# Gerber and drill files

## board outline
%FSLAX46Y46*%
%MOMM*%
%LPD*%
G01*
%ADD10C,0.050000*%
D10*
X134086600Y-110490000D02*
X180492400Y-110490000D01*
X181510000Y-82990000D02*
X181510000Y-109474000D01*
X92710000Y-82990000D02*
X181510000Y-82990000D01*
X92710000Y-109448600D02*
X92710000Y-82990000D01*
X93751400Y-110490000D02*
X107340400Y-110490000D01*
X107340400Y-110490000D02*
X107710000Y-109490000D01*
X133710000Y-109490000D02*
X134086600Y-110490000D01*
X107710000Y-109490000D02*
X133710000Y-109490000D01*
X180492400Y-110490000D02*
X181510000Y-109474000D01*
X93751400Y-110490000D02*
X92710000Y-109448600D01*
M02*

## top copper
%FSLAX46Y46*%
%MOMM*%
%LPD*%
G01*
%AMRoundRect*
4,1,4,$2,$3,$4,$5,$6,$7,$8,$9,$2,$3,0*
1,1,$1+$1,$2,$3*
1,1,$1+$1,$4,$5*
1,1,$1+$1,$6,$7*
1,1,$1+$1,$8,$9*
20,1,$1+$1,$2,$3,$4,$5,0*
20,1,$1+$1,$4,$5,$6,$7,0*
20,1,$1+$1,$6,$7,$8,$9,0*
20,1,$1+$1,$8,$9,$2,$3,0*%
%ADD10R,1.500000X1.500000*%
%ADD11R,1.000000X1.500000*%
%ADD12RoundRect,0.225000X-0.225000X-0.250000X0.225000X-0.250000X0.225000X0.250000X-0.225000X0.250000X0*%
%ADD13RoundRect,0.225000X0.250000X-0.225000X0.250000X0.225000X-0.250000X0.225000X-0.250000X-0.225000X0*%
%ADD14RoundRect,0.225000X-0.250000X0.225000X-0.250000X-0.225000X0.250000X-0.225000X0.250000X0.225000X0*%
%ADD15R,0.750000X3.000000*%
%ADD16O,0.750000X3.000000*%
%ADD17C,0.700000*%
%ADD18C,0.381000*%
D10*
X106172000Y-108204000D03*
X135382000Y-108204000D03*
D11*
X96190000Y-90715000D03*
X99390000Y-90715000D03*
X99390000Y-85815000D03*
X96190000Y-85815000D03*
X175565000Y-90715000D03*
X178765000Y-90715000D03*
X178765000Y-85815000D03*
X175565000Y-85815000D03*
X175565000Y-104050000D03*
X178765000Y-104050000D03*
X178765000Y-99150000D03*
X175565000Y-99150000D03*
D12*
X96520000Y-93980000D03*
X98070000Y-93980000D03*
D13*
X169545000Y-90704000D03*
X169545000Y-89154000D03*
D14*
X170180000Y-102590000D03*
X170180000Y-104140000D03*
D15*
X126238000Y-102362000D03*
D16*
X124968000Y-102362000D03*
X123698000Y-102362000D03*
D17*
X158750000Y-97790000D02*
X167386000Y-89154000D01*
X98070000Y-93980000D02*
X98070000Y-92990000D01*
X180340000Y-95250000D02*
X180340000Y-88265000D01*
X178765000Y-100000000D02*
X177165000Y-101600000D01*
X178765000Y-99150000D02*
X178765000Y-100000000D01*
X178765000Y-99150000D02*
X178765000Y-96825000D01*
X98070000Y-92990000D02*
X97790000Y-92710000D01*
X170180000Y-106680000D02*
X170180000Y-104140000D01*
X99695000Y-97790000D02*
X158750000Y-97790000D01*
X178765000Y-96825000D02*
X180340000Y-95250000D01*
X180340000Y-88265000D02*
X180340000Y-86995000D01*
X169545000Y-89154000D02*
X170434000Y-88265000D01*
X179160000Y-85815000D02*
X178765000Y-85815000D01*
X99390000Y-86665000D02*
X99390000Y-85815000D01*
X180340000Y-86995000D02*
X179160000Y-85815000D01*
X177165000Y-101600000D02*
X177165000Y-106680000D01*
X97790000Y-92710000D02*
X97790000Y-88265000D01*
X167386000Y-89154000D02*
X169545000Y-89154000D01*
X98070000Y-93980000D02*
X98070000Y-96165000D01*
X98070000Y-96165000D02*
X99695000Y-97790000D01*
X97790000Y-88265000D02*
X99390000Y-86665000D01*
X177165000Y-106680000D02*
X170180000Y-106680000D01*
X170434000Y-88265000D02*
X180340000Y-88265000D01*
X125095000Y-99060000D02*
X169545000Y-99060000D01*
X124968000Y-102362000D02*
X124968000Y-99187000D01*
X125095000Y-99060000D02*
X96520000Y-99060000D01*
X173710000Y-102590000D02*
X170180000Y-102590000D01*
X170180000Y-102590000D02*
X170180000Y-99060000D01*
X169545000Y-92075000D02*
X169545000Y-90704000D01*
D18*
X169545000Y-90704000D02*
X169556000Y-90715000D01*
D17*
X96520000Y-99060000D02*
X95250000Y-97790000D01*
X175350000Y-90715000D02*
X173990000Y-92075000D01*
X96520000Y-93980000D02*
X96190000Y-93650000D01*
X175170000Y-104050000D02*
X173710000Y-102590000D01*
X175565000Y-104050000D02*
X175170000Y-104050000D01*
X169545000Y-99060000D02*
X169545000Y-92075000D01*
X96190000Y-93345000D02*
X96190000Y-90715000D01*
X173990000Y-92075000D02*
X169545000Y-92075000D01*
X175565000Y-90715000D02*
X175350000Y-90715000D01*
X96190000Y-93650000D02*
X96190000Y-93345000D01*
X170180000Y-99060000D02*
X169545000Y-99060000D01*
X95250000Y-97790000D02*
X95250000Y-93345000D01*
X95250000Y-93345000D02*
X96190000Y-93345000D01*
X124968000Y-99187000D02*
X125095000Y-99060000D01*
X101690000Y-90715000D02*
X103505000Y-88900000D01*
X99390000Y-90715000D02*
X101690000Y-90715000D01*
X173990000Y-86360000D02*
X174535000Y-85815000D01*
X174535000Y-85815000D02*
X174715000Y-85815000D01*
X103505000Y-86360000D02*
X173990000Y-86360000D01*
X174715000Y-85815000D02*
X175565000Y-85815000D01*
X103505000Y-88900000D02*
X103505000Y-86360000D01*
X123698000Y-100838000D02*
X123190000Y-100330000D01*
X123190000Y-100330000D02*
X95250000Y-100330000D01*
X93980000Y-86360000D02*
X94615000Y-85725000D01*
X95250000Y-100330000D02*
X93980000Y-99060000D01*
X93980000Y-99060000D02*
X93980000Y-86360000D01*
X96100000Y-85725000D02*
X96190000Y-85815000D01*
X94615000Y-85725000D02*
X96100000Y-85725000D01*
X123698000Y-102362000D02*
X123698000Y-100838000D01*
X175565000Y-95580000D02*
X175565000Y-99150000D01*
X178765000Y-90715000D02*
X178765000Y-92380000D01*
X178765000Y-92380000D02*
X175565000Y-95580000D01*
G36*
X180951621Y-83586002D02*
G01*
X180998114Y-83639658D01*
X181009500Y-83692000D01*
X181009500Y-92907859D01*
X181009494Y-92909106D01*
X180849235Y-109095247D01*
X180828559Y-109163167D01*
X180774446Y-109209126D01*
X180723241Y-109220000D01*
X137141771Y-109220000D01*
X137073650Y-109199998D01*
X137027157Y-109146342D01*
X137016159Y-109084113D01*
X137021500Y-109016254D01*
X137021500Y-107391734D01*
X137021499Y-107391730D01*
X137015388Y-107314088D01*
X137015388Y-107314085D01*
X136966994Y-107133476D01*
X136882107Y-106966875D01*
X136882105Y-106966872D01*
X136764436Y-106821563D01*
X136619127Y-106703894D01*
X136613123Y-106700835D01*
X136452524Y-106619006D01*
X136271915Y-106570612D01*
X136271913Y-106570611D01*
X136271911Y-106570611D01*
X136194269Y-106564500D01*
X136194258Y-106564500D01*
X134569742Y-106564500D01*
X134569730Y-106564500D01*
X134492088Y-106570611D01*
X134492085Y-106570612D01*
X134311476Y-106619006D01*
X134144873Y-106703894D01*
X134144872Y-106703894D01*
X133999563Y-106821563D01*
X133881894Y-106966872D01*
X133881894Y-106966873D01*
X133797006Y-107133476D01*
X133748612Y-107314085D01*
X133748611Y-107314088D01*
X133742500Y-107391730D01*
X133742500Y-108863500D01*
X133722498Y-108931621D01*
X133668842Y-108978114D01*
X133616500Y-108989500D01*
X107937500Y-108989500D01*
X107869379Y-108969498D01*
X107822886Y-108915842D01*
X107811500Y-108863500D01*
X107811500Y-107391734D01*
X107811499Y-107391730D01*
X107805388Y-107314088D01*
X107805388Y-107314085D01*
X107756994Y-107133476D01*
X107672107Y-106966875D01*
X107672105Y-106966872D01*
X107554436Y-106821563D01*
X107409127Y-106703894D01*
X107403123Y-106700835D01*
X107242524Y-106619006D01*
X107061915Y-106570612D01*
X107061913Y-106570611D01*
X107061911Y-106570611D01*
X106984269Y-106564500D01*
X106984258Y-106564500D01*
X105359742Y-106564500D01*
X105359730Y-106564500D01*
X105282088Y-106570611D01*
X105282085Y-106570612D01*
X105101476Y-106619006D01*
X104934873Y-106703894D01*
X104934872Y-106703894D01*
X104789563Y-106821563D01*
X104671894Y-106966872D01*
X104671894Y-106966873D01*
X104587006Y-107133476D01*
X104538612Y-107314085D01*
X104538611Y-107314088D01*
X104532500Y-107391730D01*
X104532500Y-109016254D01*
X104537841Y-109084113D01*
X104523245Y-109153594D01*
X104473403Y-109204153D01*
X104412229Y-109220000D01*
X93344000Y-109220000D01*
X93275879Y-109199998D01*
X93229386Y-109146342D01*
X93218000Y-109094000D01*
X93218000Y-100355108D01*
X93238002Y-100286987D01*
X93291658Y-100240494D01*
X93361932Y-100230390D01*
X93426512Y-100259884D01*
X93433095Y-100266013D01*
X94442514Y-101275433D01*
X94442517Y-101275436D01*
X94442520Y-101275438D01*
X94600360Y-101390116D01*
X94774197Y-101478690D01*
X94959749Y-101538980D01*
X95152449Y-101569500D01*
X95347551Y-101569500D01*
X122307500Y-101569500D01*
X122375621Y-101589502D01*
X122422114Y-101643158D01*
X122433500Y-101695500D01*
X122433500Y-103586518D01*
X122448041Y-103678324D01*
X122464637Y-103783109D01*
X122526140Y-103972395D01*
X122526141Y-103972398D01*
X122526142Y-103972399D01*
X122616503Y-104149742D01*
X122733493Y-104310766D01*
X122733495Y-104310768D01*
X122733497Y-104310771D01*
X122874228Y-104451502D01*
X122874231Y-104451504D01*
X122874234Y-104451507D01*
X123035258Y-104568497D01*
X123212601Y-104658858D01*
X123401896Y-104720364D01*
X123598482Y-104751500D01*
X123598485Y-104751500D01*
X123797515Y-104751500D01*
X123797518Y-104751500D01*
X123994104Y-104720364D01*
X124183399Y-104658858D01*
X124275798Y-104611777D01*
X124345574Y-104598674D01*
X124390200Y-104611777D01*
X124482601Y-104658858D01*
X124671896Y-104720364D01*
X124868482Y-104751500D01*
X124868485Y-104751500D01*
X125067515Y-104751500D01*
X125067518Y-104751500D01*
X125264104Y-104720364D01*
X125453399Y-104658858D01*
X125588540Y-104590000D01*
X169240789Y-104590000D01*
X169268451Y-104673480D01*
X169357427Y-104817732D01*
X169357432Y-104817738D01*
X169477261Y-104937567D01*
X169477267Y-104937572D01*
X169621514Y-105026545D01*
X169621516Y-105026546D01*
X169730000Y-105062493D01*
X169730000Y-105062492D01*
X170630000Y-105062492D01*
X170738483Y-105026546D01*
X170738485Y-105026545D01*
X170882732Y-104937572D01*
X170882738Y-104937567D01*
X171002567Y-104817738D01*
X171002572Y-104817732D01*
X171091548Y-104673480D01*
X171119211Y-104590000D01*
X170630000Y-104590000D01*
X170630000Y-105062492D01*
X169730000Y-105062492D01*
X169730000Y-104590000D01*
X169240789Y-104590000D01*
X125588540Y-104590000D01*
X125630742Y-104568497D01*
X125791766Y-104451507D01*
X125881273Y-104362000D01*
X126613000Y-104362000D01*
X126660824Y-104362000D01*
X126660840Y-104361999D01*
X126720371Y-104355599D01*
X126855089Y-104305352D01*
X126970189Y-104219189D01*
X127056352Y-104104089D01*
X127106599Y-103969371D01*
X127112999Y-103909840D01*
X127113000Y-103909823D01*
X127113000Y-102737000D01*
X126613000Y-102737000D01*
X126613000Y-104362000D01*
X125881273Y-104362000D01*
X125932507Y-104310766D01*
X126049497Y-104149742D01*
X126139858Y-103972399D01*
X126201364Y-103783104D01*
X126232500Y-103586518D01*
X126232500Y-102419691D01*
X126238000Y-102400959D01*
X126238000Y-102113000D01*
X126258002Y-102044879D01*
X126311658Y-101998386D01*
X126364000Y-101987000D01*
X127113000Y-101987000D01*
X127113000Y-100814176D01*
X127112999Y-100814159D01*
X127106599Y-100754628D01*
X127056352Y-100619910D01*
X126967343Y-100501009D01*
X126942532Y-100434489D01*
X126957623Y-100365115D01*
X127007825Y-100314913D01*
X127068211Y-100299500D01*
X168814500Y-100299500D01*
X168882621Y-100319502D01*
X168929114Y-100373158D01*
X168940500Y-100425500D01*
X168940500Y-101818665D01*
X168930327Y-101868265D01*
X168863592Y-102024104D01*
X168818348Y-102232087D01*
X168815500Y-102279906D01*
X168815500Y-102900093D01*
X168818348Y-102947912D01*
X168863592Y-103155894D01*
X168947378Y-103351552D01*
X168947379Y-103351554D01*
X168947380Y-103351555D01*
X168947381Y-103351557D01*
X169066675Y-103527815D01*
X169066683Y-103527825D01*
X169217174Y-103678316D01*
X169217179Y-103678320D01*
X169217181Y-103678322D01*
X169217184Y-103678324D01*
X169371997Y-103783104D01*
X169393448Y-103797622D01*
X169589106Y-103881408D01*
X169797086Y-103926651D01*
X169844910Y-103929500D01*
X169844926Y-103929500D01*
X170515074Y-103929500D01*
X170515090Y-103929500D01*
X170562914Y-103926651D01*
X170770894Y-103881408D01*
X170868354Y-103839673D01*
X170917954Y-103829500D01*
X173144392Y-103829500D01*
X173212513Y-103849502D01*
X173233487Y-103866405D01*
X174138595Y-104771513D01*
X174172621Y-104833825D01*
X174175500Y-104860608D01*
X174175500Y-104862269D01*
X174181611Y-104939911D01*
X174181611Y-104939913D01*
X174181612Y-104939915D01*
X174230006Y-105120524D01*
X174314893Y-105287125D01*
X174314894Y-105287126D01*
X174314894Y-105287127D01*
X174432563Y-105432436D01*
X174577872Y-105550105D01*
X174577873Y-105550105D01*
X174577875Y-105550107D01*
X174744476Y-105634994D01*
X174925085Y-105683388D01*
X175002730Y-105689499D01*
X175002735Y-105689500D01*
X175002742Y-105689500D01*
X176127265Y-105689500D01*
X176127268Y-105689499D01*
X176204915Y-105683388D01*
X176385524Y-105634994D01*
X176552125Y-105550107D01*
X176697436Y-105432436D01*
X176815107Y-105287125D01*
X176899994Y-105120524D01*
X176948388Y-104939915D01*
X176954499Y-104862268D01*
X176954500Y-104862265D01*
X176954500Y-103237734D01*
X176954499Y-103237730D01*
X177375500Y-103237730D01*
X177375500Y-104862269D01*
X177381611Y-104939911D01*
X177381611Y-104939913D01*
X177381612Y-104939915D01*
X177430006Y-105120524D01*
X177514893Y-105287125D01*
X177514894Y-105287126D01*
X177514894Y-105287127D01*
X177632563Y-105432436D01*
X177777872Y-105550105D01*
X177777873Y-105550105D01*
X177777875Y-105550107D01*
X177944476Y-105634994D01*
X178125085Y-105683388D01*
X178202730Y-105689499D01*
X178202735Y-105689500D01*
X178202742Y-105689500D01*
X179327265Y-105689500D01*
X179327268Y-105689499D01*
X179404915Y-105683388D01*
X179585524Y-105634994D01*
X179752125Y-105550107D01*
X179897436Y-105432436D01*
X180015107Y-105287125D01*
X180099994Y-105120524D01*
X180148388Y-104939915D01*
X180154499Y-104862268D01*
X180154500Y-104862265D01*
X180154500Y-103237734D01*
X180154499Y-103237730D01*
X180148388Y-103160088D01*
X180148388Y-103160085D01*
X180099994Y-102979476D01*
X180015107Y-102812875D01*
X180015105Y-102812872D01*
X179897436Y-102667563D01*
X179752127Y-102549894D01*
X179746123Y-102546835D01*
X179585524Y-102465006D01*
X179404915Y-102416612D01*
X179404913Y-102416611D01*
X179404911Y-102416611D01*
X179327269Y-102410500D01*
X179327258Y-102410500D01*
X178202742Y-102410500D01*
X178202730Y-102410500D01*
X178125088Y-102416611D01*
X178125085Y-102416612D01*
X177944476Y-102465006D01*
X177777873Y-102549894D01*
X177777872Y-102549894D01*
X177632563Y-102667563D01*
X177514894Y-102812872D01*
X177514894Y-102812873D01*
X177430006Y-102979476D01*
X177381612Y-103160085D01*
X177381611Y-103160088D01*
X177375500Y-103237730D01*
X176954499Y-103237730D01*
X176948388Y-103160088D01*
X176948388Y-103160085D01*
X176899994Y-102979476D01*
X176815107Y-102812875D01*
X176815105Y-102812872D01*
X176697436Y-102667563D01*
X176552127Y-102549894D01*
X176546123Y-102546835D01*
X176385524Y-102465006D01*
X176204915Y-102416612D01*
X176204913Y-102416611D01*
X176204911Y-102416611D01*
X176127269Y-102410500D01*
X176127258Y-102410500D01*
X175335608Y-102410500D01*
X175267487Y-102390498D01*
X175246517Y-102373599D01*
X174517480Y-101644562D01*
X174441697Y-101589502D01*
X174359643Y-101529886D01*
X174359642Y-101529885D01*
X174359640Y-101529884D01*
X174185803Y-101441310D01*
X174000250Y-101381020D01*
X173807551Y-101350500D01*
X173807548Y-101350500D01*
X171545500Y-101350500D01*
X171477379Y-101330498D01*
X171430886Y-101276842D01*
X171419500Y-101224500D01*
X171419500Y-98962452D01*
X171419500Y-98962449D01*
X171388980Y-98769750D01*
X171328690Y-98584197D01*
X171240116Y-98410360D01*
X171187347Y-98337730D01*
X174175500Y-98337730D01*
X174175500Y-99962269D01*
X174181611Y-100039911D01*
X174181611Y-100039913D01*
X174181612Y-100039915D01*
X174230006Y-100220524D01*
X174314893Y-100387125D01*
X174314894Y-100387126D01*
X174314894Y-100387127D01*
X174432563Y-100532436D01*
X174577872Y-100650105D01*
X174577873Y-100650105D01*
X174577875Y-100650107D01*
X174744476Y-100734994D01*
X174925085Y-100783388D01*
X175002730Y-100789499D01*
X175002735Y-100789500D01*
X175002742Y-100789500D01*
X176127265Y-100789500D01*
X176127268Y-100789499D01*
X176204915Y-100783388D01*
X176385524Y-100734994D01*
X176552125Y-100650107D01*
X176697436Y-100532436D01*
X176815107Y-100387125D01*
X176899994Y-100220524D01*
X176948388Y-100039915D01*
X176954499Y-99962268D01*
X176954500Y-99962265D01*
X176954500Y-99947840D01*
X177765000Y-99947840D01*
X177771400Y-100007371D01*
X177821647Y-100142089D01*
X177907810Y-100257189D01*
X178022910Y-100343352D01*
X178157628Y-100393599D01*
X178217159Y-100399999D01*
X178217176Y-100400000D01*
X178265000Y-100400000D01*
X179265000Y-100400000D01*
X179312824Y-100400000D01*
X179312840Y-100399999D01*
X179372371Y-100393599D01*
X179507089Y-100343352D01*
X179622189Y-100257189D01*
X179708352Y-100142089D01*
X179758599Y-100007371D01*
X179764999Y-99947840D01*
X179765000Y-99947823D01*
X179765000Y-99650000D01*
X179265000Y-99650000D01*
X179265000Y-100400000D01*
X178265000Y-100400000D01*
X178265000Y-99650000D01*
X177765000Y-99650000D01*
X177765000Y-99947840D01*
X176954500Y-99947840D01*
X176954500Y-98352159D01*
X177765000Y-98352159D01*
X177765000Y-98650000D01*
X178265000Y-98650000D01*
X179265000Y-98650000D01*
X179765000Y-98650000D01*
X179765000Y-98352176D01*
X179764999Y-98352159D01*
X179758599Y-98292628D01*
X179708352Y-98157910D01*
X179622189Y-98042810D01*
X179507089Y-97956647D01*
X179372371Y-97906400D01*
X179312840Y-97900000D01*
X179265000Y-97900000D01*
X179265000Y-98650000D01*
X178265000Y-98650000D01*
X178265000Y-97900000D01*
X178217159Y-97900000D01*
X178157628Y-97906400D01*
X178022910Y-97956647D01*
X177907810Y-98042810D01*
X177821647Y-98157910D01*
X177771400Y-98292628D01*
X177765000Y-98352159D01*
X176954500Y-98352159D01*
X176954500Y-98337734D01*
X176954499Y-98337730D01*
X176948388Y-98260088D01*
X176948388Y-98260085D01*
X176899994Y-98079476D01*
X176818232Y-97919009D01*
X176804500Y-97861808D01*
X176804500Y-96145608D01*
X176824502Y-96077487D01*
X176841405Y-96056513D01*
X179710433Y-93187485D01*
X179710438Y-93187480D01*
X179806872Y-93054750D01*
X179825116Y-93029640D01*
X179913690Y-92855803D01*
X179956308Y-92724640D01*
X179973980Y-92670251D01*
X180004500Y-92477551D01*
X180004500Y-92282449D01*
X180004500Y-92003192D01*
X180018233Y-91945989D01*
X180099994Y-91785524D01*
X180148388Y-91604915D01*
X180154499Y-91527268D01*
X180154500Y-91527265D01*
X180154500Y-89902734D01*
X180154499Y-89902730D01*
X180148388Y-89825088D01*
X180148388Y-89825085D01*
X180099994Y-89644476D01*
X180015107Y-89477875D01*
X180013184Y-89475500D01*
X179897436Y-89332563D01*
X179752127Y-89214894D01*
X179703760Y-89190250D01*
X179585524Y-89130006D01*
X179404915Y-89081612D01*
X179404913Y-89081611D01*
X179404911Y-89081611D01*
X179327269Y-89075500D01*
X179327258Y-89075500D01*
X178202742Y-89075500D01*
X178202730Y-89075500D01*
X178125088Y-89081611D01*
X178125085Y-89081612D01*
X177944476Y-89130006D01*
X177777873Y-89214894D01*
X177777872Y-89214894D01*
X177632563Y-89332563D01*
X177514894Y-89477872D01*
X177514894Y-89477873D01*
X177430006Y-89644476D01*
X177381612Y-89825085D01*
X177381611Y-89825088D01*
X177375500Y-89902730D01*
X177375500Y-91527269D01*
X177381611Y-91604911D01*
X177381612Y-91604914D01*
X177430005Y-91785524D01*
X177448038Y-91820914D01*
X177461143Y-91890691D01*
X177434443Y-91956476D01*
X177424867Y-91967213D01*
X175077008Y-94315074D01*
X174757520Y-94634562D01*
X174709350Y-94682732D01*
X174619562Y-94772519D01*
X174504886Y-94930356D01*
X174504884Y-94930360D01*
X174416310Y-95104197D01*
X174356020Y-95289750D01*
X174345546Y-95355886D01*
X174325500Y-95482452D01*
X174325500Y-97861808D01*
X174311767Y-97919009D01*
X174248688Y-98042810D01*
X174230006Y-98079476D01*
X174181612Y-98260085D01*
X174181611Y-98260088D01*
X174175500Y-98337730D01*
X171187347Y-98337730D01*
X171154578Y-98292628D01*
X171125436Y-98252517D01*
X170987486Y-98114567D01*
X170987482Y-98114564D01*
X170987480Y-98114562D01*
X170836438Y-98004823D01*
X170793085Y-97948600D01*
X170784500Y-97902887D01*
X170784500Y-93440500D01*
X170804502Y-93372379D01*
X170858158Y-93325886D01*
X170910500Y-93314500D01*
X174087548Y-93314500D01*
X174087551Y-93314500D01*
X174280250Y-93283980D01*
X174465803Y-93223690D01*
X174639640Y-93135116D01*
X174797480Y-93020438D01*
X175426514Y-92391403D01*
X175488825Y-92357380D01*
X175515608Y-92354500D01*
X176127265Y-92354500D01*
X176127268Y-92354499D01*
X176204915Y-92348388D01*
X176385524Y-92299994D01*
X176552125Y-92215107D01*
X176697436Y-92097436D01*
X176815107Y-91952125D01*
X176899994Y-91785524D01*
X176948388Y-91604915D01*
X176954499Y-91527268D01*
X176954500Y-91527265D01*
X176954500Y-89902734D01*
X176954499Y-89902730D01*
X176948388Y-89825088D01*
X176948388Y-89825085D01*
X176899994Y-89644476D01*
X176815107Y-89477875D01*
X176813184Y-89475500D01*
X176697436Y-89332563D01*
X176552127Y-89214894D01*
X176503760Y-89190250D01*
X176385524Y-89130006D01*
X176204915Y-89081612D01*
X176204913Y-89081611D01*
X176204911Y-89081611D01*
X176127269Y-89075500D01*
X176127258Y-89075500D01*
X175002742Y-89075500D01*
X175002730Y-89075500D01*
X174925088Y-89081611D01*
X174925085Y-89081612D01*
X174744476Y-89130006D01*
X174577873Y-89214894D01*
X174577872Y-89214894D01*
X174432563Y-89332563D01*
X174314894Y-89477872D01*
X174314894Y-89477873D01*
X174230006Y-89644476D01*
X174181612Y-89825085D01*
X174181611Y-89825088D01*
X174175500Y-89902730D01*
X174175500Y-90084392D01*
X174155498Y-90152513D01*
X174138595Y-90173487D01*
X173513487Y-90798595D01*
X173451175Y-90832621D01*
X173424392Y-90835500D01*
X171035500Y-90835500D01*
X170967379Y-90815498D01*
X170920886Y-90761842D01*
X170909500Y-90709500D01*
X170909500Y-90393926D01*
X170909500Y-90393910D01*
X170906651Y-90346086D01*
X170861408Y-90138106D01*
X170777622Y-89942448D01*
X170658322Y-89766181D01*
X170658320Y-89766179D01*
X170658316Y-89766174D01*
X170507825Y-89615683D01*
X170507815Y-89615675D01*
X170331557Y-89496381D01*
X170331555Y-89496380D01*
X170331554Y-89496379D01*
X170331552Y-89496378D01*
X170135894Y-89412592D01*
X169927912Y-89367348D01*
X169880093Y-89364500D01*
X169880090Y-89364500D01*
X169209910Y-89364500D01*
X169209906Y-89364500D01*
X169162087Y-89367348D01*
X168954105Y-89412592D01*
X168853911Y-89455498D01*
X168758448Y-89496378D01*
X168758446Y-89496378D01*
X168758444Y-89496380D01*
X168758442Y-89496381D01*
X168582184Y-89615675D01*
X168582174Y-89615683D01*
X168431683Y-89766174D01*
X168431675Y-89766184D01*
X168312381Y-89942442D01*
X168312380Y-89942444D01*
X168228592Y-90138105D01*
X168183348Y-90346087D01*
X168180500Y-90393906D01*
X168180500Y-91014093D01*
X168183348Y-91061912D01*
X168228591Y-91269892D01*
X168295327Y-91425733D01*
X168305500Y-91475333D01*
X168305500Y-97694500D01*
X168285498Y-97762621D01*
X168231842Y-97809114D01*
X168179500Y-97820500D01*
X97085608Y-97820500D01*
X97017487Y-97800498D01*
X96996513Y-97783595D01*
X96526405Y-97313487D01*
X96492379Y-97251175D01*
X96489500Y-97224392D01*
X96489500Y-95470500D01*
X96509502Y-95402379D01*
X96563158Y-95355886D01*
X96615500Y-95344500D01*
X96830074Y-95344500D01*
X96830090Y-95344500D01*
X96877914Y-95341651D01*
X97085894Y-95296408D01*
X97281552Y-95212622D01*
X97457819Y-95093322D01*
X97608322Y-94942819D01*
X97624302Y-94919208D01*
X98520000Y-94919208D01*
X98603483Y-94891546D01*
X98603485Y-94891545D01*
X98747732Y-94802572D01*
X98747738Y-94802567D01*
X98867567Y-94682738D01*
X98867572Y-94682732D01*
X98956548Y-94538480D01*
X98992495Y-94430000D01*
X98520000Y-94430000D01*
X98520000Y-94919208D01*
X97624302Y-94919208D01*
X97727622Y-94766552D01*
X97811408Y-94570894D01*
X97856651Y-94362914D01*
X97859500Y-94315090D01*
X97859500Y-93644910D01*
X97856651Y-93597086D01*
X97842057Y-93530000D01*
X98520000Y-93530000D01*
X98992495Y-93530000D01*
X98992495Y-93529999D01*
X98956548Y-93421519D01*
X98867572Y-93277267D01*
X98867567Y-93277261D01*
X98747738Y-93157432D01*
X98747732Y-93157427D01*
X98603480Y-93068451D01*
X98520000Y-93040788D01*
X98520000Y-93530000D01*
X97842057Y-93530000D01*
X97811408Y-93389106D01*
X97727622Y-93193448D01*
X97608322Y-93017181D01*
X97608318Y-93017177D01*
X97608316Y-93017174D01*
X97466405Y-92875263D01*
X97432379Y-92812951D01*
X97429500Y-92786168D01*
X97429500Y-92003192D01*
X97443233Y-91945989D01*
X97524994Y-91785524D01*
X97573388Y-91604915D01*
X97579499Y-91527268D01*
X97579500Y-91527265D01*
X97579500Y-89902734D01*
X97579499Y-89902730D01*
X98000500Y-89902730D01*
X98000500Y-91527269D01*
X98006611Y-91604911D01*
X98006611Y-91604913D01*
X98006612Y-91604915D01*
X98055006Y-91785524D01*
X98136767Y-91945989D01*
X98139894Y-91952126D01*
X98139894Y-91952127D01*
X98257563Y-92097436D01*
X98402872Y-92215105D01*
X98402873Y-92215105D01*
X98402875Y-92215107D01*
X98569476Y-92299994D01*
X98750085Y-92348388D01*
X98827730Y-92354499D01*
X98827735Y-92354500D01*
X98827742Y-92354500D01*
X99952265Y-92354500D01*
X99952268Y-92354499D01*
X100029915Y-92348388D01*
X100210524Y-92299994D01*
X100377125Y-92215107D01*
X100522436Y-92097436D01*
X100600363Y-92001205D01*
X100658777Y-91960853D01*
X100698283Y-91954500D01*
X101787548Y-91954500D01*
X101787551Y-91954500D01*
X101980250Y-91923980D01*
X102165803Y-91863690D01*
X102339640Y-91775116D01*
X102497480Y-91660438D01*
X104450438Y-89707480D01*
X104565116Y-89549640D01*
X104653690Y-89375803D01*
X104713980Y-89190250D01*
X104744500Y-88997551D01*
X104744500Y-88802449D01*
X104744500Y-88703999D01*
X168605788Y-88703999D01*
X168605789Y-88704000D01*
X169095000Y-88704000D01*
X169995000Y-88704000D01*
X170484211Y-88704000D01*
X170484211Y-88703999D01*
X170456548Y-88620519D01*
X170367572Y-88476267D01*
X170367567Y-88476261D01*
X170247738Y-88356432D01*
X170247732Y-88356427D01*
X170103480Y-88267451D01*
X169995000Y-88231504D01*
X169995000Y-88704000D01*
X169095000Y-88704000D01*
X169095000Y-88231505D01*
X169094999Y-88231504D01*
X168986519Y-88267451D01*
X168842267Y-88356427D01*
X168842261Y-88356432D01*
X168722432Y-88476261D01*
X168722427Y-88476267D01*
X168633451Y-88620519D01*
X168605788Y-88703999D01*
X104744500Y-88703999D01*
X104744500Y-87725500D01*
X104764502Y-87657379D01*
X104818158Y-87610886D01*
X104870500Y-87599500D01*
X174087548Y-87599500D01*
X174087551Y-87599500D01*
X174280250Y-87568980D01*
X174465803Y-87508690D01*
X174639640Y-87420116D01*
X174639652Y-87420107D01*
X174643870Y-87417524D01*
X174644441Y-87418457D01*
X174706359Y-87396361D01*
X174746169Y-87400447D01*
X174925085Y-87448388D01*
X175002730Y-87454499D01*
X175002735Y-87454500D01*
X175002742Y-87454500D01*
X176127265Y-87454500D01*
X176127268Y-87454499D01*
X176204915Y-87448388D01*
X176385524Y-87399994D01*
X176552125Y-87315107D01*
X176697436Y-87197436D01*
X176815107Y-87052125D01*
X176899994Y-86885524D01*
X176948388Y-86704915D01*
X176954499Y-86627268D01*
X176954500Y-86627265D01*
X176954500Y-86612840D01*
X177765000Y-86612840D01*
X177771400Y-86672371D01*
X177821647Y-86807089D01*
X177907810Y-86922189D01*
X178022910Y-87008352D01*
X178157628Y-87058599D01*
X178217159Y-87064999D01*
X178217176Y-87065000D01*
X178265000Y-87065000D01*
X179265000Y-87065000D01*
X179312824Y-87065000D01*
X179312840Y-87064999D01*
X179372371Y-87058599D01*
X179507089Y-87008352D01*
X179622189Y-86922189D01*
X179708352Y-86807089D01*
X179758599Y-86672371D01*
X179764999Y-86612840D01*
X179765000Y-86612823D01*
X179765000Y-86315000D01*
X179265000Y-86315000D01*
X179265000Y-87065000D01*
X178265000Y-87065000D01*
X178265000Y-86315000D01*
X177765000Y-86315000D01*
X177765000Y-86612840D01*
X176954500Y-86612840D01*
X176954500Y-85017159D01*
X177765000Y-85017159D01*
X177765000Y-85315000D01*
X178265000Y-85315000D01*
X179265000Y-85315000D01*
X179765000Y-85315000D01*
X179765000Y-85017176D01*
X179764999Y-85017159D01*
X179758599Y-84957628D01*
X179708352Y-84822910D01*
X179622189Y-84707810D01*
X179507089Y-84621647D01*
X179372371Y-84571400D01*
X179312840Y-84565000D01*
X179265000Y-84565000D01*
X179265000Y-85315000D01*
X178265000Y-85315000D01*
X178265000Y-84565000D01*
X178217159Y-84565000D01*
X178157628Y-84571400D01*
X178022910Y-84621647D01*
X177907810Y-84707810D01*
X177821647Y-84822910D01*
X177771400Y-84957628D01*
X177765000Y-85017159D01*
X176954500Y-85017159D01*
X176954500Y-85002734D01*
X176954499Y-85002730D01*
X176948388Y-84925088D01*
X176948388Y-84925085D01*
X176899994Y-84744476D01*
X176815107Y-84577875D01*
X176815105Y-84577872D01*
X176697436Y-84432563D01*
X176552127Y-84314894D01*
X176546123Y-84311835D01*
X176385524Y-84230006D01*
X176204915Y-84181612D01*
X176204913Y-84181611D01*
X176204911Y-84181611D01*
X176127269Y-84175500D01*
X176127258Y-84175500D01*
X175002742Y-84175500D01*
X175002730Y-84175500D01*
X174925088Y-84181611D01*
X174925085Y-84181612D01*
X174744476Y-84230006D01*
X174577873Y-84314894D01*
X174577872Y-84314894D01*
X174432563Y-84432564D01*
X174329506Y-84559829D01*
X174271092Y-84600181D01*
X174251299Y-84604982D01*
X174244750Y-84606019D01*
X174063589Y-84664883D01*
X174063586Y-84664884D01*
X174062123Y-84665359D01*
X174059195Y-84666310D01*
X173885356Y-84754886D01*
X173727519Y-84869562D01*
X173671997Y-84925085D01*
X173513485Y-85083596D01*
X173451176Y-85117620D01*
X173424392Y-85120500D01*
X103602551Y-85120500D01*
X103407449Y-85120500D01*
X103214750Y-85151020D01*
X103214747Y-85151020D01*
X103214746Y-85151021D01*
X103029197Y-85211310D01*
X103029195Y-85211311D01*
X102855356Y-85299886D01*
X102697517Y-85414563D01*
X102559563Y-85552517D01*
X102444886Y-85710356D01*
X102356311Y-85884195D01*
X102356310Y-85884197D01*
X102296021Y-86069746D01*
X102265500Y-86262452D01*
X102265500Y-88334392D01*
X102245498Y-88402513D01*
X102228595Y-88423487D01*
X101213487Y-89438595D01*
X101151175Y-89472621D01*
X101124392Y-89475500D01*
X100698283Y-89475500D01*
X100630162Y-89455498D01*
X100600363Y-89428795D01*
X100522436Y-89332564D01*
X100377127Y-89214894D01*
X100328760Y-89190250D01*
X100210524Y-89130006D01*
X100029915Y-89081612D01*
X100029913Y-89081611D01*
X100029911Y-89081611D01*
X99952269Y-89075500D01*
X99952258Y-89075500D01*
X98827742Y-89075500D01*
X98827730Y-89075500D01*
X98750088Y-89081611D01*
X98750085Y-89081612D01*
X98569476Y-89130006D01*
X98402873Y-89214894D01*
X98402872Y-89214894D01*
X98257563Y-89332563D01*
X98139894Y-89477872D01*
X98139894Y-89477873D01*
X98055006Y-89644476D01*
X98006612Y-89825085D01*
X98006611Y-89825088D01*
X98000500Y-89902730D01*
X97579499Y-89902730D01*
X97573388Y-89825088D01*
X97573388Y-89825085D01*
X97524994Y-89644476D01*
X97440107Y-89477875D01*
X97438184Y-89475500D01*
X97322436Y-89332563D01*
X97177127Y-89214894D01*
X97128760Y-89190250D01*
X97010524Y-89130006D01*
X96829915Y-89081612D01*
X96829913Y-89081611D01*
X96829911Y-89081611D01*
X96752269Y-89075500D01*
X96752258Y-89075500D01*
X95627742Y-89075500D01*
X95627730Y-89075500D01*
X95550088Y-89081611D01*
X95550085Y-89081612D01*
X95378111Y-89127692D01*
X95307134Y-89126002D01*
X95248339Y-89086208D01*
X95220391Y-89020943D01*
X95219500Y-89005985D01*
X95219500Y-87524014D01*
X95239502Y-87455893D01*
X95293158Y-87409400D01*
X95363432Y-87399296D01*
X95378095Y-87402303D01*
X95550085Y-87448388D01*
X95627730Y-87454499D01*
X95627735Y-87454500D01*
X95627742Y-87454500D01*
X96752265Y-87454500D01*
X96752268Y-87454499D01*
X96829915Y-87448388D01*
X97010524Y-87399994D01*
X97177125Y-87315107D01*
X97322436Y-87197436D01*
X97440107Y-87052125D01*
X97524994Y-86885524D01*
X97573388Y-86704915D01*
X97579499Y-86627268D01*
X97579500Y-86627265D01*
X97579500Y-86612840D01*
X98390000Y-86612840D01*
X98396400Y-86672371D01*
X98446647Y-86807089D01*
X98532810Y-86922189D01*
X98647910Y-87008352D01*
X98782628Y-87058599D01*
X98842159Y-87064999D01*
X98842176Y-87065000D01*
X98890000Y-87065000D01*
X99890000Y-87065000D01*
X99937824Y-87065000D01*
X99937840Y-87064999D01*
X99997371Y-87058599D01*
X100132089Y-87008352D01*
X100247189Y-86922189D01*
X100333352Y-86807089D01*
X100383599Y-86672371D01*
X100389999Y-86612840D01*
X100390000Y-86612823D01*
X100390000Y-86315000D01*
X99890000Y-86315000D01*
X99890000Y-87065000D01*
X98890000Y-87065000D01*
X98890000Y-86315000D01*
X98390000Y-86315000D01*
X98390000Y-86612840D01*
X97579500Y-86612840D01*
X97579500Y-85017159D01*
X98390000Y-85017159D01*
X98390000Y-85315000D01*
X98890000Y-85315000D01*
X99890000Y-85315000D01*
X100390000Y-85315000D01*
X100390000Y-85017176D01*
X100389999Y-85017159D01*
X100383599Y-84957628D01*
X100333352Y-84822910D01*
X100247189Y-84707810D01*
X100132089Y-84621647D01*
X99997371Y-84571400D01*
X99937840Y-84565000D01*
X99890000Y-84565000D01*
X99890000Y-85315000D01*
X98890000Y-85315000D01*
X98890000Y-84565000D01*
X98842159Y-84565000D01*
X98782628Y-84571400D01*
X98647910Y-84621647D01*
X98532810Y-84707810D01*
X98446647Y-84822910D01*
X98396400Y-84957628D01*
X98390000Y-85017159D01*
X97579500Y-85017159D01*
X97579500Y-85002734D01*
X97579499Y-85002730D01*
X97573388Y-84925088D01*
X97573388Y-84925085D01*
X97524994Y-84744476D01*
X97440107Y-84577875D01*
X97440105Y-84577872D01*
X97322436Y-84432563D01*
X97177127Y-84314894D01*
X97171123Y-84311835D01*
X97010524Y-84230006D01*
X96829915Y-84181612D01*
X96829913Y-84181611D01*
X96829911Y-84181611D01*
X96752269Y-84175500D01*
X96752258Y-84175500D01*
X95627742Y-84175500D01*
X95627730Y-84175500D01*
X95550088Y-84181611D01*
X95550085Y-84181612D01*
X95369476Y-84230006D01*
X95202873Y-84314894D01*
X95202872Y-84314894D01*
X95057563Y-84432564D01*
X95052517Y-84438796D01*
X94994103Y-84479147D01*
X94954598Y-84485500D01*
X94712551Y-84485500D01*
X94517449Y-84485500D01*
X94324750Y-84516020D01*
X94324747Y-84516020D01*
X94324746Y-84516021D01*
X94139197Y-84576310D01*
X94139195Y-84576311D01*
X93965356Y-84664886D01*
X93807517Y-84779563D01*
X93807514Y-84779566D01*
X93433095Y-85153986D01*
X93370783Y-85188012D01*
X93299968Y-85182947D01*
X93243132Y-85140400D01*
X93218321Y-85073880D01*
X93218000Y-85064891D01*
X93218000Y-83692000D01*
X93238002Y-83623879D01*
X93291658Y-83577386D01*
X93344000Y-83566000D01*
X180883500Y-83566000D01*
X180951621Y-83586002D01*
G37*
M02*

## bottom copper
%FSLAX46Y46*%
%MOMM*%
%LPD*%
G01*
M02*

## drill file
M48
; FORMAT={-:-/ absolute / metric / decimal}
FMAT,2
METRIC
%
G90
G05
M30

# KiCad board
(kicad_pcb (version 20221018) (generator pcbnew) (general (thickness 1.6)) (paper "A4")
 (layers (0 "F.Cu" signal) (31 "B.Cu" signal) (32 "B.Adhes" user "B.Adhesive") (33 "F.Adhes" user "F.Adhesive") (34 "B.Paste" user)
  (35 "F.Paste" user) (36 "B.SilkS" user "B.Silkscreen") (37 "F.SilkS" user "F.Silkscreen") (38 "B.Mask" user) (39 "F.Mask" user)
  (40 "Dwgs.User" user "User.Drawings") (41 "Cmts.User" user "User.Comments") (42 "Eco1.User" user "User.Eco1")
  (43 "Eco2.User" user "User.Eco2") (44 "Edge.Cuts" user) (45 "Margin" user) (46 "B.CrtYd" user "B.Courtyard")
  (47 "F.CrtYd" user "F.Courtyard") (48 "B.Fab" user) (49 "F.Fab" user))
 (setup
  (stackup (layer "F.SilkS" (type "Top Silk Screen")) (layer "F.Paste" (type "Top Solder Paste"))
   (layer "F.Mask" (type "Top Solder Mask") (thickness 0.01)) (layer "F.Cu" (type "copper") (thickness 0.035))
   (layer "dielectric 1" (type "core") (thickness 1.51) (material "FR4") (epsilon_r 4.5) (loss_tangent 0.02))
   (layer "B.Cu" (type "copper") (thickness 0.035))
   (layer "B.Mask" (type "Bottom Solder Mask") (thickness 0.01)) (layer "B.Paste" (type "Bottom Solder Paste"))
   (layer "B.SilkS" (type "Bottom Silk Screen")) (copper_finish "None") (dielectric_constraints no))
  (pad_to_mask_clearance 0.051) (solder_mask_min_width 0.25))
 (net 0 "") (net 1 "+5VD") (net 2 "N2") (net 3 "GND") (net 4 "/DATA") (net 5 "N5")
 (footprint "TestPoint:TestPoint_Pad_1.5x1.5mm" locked (layer "F.Cu") (at 106.172 108.204)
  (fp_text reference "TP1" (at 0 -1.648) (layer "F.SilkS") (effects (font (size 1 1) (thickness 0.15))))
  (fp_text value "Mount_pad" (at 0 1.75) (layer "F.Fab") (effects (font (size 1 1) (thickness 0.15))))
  (pad "1" smd rect locked (at 0 0) (size 1.5 1.5) (layers "F.Cu" "F.Mask")))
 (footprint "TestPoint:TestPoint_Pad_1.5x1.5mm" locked (layer "F.Cu") (at 135.382 108.204)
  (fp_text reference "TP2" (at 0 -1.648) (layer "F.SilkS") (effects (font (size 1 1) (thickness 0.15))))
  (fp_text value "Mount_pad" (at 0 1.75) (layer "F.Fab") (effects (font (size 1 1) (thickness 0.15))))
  (pad "1" smd rect locked (at 0 0) (size 1.5 1.5) (layers "F.Cu" "F.Mask")))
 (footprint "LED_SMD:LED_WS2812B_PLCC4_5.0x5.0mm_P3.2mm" (layer "F.Cu") (at 97.79 88.265 90)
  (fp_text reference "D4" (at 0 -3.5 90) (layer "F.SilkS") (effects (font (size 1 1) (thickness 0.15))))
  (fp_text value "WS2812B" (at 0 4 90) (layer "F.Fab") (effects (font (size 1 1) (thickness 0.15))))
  (pad "1" smd rect (at -2.45 -1.6 90) (size 1.5 1) (layers "F.Cu" "F.Paste" "F.Mask") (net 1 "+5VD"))
  (pad "2" smd rect (at -2.45 1.6 90) (size 1.5 1) (layers "F.Cu" "F.Paste" "F.Mask") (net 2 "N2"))
  (pad "3" smd rect (at 2.45 1.6 90) (size 1.5 1) (layers "F.Cu" "F.Paste" "F.Mask") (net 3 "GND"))
  (pad "4" smd rect (at 2.45 -1.6 90) (size 1.5 1) (layers "F.Cu" "F.Paste" "F.Mask") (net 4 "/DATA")))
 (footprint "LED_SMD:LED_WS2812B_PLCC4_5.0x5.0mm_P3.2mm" (layer "F.Cu") (at 177.165 88.265 90)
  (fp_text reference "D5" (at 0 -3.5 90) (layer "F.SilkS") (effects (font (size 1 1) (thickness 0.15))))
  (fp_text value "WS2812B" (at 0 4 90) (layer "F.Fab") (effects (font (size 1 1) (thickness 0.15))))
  (pad "1" smd rect (at -2.45 -1.6 90) (size 1.5 1) (layers "F.Cu" "F.Paste" "F.Mask") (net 1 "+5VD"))
  (pad "2" smd rect (at -2.45 1.6 90) (size 1.5 1) (layers "F.Cu" "F.Paste" "F.Mask") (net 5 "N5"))
  (pad "3" smd rect (at 2.45 1.6 90) (size 1.5 1) (layers "F.Cu" "F.Paste" "F.Mask") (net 3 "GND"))
  (pad "4" smd rect (at 2.45 -1.6 90) (size 1.5 1) (layers "F.Cu" "F.Paste" "F.Mask") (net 2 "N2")))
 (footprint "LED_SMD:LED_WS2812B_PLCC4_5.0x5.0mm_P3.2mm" (layer "F.Cu") (at 177.165 101.6 90)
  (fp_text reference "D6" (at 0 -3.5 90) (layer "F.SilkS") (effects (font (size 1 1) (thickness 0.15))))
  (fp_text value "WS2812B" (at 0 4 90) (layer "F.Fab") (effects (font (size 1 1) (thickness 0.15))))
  (pad "1" smd rect (at -2.45 -1.6 90) (size 1.5 1) (layers "F.Cu" "F.Paste" "F.Mask") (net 1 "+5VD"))
  (pad "2" smd rect (at -2.45 1.6 90) (size 1.5 1) (layers "F.Cu" "F.Paste" "F.Mask"))
  (pad "3" smd rect (at 2.45 1.6 90) (size 1.5 1) (layers "F.Cu" "F.Paste" "F.Mask") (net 3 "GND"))
  (pad "4" smd rect (at 2.45 -1.6 90) (size 1.5 1) (layers "F.Cu" "F.Paste" "F.Mask") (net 5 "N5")))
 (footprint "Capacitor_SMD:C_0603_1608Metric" (layer "F.Cu") (at 97.295 93.98)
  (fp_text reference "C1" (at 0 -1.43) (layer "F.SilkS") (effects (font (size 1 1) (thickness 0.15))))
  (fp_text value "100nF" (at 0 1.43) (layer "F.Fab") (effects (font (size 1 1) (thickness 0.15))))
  (pad "1" smd roundrect (at -0.775 0) (size 0.9 0.95) (layers "F.Cu" "F.Paste" "F.Mask") (roundrect_rratio 0.25) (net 1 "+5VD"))
  (pad "2" smd roundrect (at 0.775 0) (size 0.9 0.95) (layers "F.Cu" "F.Paste" "F.Mask") (roundrect_rratio 0.25) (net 3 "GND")))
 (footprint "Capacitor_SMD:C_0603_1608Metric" (layer "F.Cu") (at 169.545 89.929 90)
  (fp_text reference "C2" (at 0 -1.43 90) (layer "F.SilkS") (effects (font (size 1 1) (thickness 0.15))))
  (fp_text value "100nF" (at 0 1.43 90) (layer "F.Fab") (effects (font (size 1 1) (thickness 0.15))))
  (pad "1" smd roundrect (at -0.775 0 90) (size 0.9 0.95) (layers "F.Cu" "F.Paste" "F.Mask") (roundrect_rratio 0.25) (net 1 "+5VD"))
  (pad "2" smd roundrect (at 0.775 0 90) (size 0.9 0.95) (layers "F.Cu" "F.Paste" "F.Mask") (roundrect_rratio 0.25) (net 3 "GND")))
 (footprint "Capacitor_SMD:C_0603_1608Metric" (layer "F.Cu") (at 170.18 103.365 -90)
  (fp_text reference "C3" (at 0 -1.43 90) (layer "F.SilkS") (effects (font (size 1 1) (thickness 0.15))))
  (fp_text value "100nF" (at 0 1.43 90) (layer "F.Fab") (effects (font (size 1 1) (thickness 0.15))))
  (pad "1" smd roundrect (at -0.775 0 270) (size 0.9 0.95) (layers "F.Cu" "F.Paste" "F.Mask") (roundrect_rratio 0.25) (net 1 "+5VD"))
  (pad "2" smd roundrect (at 0.775 0 270) (size 0.9 0.95) (layers "F.Cu" "F.Paste" "F.Mask") (roundrect_rratio 0.25) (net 3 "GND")))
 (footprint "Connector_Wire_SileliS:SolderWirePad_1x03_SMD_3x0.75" (layer "F.Cu") (at 124.9553 105.3493 180)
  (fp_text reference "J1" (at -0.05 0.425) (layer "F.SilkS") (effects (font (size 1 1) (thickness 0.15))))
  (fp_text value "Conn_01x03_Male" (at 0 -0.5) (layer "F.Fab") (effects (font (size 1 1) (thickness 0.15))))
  (pad "1" smd rect (at -1.2827 2.9873 180) (size 0.75 3) (layers "F.Cu" "F.Mask") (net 3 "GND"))
  (pad "2" smd oval (at -0.0127 2.9873 180) (size 0.75 3) (layers "F.Cu" "F.Mask") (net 1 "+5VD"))
  (pad "3" smd oval (at 1.2573 2.9873 180) (size 0.75 3) (layers "F.Cu" "F.Mask") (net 4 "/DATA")))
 (gr_line (start 134.0866 110.49) (end 180.4924 110.49) (stroke (width 0.05) (type solid)) (layer "Edge.Cuts"))
 (gr_line (start 181.51 82.99) (end 181.51 109.474) (stroke (width 0.05) (type solid)) (layer "Edge.Cuts"))
 (gr_line (start 92.71 82.99) (end 181.51 82.99) (stroke (width 0.05) (type solid)) (layer "Edge.Cuts"))
 (gr_line (start 92.71 109.4486) (end 92.71 82.99) (stroke (width 0.05) (type solid)) (layer "Edge.Cuts"))
 (gr_line (start 93.7514 110.49) (end 107.3404 110.49) (stroke (width 0.05) (type solid)) (layer "Edge.Cuts"))
 (gr_line (start 107.3404 110.49) (end 107.71 109.49) (stroke (width 0.05) (type solid)) (layer "Edge.Cuts"))
 (gr_line (start 133.71 109.49) (end 134.0866 110.49) (stroke (width 0.05) (type solid)) (layer "Edge.Cuts"))
 (gr_line (start 107.71 109.49) (end 133.71 109.49) (stroke (width 0.05) (type solid)) (layer "Edge.Cuts"))
 (gr_line (start 180.4924 110.49) (end 181.51 109.474) (stroke (width 0.05) (type solid)) (layer "Edge.Cuts"))
 (gr_line (start 93.7514 110.49) (end 92.71 109.4486) (stroke (width 0.05) (type solid)) (layer "Edge.Cuts"))
 (segment (start 158.75 97.79) (end 167.386 89.154) (width 0.7) (layer "F.Cu") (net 3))
 (segment (start 98.07 93.98) (end 98.07 92.99) (width 0.7) (layer "F.Cu") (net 3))
 (segment (start 180.34 95.25) (end 180.34 88.265) (width 0.7) (layer "F.Cu") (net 3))
 (segment (start 178.765 100) (end 177.165 101.6) (width 0.7) (layer "F.Cu") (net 3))
 (segment (start 178.765 99.15) (end 178.765 100) (width 0.7) (layer "F.Cu") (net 3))
 (segment (start 178.765 99.15) (end 178.765 96.825) (width 0.7) (layer "F.Cu") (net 3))
 (segment (start 98.07 92.99) (end 97.79 92.71) (width 0.7) (layer "F.Cu") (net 3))
 (segment (start 170.18 106.68) (end 170.18 104.14) (width 0.7) (layer "F.Cu") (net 3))
 (segment (start 99.695 97.79) (end 158.75 97.79) (width 0.7) (layer "F.Cu") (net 3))
 (segment (start 178.765 96.825) (end 180.34 95.25) (width 0.7) (layer "F.Cu") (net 3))
 (segment (start 180.34 88.265) (end 180.34 86.995) (width 0.7) (layer "F.Cu") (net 3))
 (segment (start 169.545 89.154) (end 170.434 88.265) (width 0.7) (layer "F.Cu") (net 3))
 (segment (start 179.16 85.815) (end 178.765 85.815) (width 0.7) (layer "F.Cu") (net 3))
 (segment (start 99.39 86.665) (end 99.39 85.815) (width 0.7) (layer "F.Cu") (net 3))
 (segment (start 180.34 86.995) (end 179.16 85.815) (width 0.7) (layer "F.Cu") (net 3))
 (segment (start 177.165 101.6) (end 177.165 106.68) (width 0.7) (layer "F.Cu") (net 3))
 (segment (start 97.79 92.71) (end 97.79 88.265) (width 0.7) (layer "F.Cu") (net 3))
 (segment (start 167.386 89.154) (end 169.545 89.154) (width 0.7) (layer "F.Cu") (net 3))
 (segment (start 98.07 93.98) (end 98.07 96.165) (width 0.7) (layer "F.Cu") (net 3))
 (segment (start 98.07 96.165) (end 99.695 97.79) (width 0.7) (layer "F.Cu") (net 3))
 (segment (start 97.79 88.265) (end 99.39 86.665) (width 0.7) (layer "F.Cu") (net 3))
 (segment (start 177.165 106.68) (end 170.18 106.68) (width 0.7) (layer "F.Cu") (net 3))
 (segment (start 170.434 88.265) (end 180.34 88.265) (width 0.7) (layer "F.Cu") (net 3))
 (segment (start 125.095 99.06) (end 169.545 99.06) (width 0.7) (layer "F.Cu") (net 1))
 (segment (start 124.968 102.362) (end 124.968 99.187) (width 0.7) (layer "F.Cu") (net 1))
 (segment (start 125.095 99.06) (end 96.52 99.06) (width 0.7) (layer "F.Cu") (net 1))
 (segment (start 173.71 102.59) (end 170.18 102.59) (width 0.7) (layer "F.Cu") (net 1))
 (segment (start 170.18 102.59) (end 170.18 99.06) (width 0.7) (layer "F.Cu") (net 1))
 (segment (start 169.545 92.075) (end 169.545 90.704) (width 0.7) (layer "F.Cu") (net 1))
 (segment (start 169.545 90.704) (end 169.556 90.715) (width 0.381) (layer "F.Cu") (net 1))
 (segment (start 96.52 99.06) (end 95.25 97.79) (width 0.7) (layer "F.Cu") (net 1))
 (segment (start 175.35 90.715) (end 173.99 92.075) (width 0.7) (layer "F.Cu") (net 1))
 (segment (start 96.52 93.98) (end 96.19 93.65) (width 0.7) (layer "F.Cu") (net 1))
 (segment (start 175.17 104.05) (end 173.71 102.59) (width 0.7) (layer "F.Cu") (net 1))
 (segment (start 175.565 104.05) (end 175.17 104.05) (width 0.7) (layer "F.Cu") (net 1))
 (segment (start 169.545 99.06) (end 169.545 92.075) (width 0.7) (layer "F.Cu") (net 1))
 (segment (start 96.19 93.345) (end 96.19 90.715) (width 0.7) (layer "F.Cu") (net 1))
 (segment (start 173.99 92.075) (end 169.545 92.075) (width 0.7) (layer "F.Cu") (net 1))
 (segment (start 175.565 90.715) (end 175.35 90.715) (width 0.7) (layer "F.Cu") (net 1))
 (segment (start 96.19 93.65) (end 96.19 93.345) (width 0.7) (layer "F.Cu") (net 1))
 (segment (start 170.18 99.06) (end 169.545 99.06) (width 0.7) (layer "F.Cu") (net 1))
 (segment (start 95.25 97.79) (end 95.25 93.345) (width 0.7) (layer "F.Cu") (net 1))
 (segment (start 95.25 93.345) (end 96.19 93.345) (width 0.7) (layer "F.Cu") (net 1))
 (segment (start 124.968 99.187) (end 125.095 99.06) (width 0.7) (layer "F.Cu") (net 1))
 (segment (start 101.69 90.715) (end 103.505 88.9) (width 0.7) (layer "F.Cu") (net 2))
 (segment (start 99.39 90.715) (end 101.69 90.715) (width 0.7) (layer "F.Cu") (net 2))
 (segment (start 173.99 86.36) (end 174.535 85.815) (width 0.7) (layer "F.Cu") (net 2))
 (segment (start 174.535 85.815) (end 174.715 85.815) (width 0.7) (layer "F.Cu") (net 2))
 (segment (start 103.505 86.36) (end 173.99 86.36) (width 0.7) (layer "F.Cu") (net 2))
 (segment (start 174.715 85.815) (end 175.565 85.815) (width 0.7) (layer "F.Cu") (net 2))
 (segment (start 103.505 88.9) (end 103.505 86.36) (width 0.7) (layer "F.Cu") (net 2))
 (segment (start 123.698 100.838) (end 123.19 100.33) (width 0.7) (layer "F.Cu") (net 4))
 (segment (start 123.19 100.33) (end 95.25 100.33) (width 0.7) (layer "F.Cu") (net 4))
 (segment (start 93.98 86.36) (end 94.615 85.725) (width 0.7) (layer "F.Cu") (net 4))
 (segment (start 95.25 100.33) (end 93.98 99.06) (width 0.7) (layer "F.Cu") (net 4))
 (segment (start 93.98 99.06) (end 93.98 86.36) (width 0.7) (layer "F.Cu") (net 4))
 (segment (start 96.1 85.725) (end 96.19 85.815) (width 0.7) (layer "F.Cu") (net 4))
 (segment (start 94.615 85.725) (end 96.1 85.725) (width 0.7) (layer "F.Cu") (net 4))
 (segment (start 123.698 102.362) (end 123.698 100.838) (width 0.7) (layer "F.Cu") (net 4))
 (segment (start 175.565 95.58) (end 175.565 99.15) (width 0.7) (layer "F.Cu") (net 5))
 (segment (start 178.765 90.715) (end 178.765 92.38) (width 0.7) (layer "F.Cu") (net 5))
 (segment (start 178.765 92.38) (end 175.565 95.58) (width 0.7) (layer "F.Cu") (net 5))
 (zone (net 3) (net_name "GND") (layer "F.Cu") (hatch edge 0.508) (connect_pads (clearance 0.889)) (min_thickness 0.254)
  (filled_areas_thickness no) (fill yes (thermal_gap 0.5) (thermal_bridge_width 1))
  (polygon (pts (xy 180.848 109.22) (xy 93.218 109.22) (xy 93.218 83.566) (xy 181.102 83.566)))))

